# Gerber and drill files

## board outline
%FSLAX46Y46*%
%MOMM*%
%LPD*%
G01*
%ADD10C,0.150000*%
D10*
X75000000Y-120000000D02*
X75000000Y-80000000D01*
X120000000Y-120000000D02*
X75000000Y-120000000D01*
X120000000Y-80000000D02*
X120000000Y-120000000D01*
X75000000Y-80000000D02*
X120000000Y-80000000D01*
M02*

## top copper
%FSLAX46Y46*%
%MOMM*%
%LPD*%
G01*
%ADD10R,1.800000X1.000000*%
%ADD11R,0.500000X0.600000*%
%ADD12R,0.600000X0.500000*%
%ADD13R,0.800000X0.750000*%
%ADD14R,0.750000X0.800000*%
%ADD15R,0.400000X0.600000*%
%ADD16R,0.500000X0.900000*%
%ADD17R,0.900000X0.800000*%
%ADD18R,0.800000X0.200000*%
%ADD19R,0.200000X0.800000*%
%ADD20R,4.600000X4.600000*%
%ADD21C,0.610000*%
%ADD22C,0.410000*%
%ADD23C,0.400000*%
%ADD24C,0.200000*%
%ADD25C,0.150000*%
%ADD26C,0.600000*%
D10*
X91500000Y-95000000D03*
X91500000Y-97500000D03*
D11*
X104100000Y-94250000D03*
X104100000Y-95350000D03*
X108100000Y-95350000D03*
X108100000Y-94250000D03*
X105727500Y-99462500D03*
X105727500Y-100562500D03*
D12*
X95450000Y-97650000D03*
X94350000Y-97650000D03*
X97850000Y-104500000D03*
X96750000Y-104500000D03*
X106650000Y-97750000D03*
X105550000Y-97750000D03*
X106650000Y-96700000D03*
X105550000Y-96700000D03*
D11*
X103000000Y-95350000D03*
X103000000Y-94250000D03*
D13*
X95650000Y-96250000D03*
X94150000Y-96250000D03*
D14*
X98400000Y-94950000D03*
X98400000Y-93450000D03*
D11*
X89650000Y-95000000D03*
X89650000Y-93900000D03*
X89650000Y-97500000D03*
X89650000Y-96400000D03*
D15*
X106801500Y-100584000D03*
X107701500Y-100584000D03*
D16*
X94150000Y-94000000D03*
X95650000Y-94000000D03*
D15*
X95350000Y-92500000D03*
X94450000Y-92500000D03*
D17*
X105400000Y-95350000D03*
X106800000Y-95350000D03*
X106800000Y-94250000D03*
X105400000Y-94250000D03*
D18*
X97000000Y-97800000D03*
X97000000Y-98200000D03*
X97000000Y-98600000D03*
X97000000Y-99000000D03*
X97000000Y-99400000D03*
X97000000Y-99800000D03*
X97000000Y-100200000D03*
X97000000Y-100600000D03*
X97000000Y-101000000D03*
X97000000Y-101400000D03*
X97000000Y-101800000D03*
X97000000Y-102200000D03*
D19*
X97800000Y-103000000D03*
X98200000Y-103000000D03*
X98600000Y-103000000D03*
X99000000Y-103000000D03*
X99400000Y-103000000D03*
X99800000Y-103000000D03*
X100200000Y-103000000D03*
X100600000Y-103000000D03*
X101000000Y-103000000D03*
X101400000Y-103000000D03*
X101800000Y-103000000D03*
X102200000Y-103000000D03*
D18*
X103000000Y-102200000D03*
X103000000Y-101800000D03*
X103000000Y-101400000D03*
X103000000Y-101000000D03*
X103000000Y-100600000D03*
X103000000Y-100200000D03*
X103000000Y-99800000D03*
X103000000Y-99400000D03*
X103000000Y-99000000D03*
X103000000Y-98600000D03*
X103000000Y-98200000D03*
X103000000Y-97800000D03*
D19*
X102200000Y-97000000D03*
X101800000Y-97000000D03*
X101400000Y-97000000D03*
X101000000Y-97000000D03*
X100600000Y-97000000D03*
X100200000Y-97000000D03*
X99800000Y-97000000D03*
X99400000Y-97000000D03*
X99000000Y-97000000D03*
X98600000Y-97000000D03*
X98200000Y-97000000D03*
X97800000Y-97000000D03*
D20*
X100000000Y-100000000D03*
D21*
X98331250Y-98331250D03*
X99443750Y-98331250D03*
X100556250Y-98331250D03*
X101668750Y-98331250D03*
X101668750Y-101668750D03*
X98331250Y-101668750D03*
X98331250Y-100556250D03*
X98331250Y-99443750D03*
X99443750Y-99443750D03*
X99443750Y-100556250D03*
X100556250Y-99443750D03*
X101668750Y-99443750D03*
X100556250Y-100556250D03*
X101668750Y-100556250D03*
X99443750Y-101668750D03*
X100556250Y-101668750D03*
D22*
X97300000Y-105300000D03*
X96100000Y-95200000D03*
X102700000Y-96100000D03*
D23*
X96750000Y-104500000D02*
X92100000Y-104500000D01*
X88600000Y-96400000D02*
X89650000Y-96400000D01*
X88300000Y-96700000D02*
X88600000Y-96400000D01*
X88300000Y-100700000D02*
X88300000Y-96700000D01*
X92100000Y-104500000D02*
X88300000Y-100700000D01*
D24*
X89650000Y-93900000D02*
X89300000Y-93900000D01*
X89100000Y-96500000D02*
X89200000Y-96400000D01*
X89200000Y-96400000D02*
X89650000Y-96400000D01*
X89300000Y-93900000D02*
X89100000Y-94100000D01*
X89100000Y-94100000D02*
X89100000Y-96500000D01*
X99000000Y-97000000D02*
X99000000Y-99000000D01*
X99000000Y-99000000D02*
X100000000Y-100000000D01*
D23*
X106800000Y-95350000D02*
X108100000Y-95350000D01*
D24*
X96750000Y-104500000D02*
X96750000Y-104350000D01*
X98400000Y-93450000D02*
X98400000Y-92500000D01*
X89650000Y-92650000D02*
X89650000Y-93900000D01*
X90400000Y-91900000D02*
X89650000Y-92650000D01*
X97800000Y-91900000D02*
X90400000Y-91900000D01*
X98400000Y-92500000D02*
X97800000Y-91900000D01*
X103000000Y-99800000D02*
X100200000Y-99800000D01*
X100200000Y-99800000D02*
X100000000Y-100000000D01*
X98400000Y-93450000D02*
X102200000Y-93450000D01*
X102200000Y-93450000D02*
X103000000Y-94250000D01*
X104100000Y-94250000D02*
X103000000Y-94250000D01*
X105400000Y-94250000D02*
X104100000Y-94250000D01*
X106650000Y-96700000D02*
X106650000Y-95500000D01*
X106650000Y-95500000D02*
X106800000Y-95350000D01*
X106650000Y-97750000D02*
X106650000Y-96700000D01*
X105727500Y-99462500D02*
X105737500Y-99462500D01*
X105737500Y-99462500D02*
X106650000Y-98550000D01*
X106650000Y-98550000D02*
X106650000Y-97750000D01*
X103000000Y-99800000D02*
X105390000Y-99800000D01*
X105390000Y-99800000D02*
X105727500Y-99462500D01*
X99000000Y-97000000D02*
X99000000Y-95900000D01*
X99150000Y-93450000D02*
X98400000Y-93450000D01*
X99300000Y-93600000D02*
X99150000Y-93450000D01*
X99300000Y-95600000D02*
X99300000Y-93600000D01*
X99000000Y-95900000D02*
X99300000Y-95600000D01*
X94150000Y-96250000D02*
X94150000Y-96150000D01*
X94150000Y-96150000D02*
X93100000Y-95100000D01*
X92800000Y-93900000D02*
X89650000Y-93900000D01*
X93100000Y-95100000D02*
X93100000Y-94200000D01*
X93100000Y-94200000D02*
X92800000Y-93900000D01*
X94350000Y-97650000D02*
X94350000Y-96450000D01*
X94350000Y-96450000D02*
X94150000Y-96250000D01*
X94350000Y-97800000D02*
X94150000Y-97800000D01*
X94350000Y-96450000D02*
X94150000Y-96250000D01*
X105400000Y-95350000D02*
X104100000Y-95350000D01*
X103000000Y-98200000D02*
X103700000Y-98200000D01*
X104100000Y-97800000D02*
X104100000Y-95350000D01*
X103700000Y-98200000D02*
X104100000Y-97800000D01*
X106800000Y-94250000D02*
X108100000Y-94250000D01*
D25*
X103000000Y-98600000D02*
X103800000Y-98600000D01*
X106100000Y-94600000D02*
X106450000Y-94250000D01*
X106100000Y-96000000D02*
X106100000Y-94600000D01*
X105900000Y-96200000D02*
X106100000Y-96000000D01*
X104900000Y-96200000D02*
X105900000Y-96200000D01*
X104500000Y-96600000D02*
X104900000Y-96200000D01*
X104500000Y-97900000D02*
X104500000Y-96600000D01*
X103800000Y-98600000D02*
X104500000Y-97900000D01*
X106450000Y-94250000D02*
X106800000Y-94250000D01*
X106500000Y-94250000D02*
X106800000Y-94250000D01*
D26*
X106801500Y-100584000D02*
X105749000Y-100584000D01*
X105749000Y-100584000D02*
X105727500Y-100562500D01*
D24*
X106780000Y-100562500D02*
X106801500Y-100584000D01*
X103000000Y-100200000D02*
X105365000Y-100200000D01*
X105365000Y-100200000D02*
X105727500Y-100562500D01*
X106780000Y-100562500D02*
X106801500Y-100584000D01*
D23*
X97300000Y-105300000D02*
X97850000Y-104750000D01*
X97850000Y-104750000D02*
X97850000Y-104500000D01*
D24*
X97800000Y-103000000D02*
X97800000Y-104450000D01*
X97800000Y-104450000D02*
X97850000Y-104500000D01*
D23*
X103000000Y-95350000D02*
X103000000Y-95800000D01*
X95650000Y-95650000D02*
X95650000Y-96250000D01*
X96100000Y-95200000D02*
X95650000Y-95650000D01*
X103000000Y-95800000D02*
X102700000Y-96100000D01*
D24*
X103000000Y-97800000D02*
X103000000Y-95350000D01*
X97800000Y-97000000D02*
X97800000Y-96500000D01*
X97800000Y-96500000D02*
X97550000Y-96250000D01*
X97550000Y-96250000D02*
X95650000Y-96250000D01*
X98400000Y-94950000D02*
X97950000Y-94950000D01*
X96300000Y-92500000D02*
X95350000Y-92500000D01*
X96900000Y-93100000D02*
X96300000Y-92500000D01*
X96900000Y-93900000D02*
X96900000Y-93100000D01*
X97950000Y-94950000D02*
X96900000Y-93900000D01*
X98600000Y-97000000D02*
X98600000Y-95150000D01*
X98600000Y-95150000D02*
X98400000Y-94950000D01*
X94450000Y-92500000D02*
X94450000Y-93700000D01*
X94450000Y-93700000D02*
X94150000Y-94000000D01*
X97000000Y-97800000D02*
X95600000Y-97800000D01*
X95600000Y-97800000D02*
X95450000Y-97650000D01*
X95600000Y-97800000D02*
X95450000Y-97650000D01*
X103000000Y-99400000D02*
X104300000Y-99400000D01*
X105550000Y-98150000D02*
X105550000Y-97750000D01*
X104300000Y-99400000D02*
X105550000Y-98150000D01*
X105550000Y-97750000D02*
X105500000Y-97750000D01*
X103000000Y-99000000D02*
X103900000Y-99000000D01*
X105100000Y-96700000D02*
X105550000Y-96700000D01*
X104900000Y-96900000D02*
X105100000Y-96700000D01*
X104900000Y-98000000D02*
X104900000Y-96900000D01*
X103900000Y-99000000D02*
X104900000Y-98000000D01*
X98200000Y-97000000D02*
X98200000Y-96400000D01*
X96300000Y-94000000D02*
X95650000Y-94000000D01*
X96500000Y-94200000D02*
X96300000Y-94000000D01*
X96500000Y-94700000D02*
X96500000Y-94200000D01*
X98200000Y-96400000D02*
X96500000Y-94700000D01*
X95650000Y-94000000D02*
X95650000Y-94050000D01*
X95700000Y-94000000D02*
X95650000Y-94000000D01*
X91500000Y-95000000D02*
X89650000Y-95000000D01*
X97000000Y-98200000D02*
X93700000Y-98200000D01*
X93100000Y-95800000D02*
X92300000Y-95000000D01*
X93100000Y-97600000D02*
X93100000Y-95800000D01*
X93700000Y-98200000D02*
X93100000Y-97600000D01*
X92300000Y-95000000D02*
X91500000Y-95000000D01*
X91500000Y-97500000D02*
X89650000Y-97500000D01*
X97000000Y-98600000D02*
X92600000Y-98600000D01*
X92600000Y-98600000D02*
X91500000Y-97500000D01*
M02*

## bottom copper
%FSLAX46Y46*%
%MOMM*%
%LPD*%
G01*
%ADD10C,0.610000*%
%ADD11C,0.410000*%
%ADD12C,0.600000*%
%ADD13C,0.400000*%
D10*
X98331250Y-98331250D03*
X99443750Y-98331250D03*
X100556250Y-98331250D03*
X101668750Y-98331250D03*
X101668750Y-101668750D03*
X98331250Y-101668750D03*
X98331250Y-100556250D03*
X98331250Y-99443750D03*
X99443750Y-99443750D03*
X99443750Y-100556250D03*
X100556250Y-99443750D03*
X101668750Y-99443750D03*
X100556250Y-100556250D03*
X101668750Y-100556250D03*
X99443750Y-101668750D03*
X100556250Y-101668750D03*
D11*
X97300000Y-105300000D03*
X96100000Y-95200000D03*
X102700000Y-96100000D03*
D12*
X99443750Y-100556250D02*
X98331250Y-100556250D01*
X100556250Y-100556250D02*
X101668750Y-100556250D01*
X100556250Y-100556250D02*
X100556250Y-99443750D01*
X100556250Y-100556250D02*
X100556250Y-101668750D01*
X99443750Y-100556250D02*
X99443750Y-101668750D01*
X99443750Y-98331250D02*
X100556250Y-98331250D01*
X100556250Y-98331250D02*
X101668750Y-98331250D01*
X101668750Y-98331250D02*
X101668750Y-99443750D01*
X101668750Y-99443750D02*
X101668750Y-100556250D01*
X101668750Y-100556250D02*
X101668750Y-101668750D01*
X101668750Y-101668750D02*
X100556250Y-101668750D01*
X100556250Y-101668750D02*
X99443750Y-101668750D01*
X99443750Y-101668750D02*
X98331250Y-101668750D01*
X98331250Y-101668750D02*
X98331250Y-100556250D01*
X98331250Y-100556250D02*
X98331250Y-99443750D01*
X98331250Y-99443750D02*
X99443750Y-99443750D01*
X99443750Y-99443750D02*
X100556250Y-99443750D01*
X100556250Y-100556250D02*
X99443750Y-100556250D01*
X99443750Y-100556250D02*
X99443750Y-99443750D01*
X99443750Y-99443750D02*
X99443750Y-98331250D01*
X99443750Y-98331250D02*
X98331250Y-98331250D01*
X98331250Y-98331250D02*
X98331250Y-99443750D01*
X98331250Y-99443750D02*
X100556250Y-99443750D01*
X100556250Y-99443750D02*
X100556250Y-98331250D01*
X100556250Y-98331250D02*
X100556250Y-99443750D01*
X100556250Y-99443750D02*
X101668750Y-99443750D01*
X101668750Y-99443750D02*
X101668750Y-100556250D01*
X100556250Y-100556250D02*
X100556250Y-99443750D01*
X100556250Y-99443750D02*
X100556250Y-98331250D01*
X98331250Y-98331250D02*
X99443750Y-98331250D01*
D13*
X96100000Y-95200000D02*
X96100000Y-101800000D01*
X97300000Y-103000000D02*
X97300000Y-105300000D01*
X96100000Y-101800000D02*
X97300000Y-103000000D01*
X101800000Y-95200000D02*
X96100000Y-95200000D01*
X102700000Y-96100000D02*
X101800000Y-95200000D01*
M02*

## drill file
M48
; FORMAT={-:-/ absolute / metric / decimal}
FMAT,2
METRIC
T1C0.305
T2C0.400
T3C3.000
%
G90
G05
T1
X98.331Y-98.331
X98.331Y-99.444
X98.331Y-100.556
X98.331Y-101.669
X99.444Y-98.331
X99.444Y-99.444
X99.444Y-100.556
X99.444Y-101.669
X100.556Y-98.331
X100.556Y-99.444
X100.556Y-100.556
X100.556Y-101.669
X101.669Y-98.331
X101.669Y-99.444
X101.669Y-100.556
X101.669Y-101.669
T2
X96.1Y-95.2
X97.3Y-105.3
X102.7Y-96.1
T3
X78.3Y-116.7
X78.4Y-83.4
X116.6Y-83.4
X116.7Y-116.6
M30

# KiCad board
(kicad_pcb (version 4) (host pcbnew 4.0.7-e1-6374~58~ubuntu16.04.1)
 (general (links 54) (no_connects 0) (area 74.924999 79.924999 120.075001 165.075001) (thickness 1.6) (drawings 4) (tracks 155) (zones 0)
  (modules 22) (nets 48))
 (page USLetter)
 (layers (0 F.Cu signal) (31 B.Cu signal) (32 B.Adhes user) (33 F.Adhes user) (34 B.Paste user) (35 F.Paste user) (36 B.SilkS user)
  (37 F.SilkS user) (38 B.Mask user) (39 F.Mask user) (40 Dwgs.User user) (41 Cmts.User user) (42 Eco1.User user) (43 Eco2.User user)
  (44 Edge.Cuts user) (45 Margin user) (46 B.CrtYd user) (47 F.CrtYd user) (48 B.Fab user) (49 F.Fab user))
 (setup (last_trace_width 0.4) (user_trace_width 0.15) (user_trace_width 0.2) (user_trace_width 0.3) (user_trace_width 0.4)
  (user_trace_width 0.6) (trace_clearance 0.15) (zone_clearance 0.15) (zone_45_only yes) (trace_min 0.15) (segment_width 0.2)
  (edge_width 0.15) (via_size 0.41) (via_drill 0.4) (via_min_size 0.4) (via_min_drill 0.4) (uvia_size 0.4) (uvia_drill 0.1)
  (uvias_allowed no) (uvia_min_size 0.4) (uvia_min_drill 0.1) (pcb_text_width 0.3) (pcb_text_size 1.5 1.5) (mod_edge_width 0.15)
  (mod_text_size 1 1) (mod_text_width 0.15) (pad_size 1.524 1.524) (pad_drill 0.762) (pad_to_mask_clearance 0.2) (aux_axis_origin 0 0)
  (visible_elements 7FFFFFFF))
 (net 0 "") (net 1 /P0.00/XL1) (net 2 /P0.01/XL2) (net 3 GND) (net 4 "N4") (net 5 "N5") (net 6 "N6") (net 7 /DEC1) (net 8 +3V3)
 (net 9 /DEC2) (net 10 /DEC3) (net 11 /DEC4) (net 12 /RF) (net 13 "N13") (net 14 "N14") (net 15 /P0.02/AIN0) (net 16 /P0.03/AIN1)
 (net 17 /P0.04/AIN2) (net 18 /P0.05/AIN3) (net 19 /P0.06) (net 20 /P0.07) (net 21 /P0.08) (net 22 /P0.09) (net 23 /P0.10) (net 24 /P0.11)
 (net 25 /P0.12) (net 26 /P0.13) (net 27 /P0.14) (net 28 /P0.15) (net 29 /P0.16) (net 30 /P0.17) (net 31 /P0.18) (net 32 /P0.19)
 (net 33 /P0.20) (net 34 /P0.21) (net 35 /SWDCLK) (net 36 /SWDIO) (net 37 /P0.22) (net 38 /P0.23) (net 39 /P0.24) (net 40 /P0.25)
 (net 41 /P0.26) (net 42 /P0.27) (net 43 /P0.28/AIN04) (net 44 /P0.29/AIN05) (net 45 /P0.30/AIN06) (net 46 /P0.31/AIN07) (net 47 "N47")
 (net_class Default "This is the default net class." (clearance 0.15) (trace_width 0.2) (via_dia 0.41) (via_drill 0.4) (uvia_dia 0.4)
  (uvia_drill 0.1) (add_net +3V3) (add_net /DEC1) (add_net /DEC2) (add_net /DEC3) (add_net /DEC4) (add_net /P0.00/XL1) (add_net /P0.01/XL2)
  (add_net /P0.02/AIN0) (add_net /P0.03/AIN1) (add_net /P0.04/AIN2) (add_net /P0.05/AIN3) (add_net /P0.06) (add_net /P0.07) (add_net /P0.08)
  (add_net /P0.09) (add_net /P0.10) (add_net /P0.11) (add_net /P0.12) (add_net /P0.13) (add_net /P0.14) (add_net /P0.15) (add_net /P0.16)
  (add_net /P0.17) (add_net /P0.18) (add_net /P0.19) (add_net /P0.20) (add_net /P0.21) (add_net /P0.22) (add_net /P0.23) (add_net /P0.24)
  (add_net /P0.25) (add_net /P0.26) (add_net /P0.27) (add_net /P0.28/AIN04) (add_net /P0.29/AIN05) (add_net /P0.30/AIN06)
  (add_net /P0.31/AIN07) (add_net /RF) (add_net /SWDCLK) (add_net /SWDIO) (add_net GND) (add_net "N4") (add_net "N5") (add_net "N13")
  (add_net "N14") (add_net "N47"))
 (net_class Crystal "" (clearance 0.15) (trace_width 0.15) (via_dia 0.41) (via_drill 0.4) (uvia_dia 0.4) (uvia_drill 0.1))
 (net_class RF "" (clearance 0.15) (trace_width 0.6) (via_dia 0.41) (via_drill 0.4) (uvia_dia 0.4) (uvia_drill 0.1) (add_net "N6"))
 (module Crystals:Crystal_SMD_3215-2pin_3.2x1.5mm (layer F.Cu) (at 91.5 96.25 90)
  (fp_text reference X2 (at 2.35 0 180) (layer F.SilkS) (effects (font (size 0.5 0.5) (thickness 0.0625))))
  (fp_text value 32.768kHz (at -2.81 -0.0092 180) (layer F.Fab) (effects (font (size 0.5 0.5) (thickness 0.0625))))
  (pad 1 smd rect (at 1.25 0 90) (size 1 1.8) (layers F.Cu F.Paste F.Mask) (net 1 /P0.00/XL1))
  (pad 2 smd rect (at -1.25 0 90) (size 1 1.8) (layers F.Cu F.Paste F.Mask) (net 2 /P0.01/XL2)))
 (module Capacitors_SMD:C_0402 (layer F.Cu) (at 104.1 94.8 270)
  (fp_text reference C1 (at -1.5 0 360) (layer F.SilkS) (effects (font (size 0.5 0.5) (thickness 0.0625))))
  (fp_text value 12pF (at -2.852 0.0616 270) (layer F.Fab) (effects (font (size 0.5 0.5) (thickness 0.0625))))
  (pad 1 smd rect (at -0.55 0 270) (size 0.6 0.5) (layers F.Cu F.Paste F.Mask) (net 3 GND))
  (pad 2 smd rect (at 0.55 0 270) (size 0.6 0.5) (layers F.Cu F.Paste F.Mask) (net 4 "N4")))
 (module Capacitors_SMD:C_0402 (layer F.Cu) (at 108.1 94.8 90)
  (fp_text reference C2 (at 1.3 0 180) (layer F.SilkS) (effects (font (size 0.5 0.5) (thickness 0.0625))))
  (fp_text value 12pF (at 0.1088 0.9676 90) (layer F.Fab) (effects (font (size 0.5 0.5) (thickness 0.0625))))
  (pad 1 smd rect (at -0.55 0 90) (size 0.6 0.5) (layers F.Cu F.Paste F.Mask) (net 3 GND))
  (pad 2 smd rect (at 0.55 0 90) (size 0.6 0.5) (layers F.Cu F.Paste F.Mask) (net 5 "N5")))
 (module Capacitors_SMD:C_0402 (layer F.Cu) (at 105.7275 100.0125 270)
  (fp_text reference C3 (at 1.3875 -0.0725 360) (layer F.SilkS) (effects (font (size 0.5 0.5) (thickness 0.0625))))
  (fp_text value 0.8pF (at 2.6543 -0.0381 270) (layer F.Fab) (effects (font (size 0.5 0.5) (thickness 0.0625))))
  (pad 1 smd rect (at -0.55 0 270) (size 0.6 0.5) (layers F.Cu F.Paste F.Mask) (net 3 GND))
  (pad 2 smd rect (at 0.55 0 270) (size 0.6 0.5) (layers F.Cu F.Paste F.Mask) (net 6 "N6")))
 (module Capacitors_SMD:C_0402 (layer F.Cu) (at 94.9 97.65 180)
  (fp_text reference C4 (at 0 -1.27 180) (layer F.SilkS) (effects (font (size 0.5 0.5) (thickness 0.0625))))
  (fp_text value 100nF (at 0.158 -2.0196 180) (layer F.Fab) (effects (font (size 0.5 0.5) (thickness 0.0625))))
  (pad 1 smd rect (at -0.55 0 180) (size 0.6 0.5) (layers F.Cu F.Paste F.Mask) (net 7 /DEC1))
  (pad 2 smd rect (at 0.55 0 180) (size 0.6 0.5) (layers F.Cu F.Paste F.Mask) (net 3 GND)))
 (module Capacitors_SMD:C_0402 (layer F.Cu) (at 97.3 104.5 180)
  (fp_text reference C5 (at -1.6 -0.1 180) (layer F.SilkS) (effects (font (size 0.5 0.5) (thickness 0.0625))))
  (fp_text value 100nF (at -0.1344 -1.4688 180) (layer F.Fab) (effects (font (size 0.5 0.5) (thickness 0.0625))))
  (pad 1 smd rect (at -0.55 0 180) (size 0.6 0.5) (layers F.Cu F.Paste F.Mask) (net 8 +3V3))
  (pad 2 smd rect (at 0.55 0 180) (size 0.6 0.5) (layers F.Cu F.Paste F.Mask) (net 3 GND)))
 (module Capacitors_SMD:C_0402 (layer F.Cu) (at 106.1 97.75 180)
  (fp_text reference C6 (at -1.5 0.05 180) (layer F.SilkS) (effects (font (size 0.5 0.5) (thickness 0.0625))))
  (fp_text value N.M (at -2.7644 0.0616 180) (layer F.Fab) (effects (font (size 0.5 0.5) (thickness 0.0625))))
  (pad 1 smd rect (at -0.55 0 180) (size 0.6 0.5) (layers F.Cu F.Paste F.Mask) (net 3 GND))
  (pad 2 smd rect (at 0.55 0 180) (size 0.6 0.5) (layers F.Cu F.Paste F.Mask) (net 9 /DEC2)))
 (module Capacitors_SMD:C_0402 (layer F.Cu) (at 106.1 96.7 180)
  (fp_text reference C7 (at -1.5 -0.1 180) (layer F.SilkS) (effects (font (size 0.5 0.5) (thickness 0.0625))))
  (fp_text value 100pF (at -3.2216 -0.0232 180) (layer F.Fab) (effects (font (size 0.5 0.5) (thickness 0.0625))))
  (pad 1 smd rect (at -0.55 0 180) (size 0.6 0.5) (layers F.Cu F.Paste F.Mask) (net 3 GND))
  (pad 2 smd rect (at 0.55 0 180) (size 0.6 0.5) (layers F.Cu F.Paste F.Mask) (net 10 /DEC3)))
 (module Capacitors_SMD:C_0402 (layer F.Cu) (at 103 94.8 90)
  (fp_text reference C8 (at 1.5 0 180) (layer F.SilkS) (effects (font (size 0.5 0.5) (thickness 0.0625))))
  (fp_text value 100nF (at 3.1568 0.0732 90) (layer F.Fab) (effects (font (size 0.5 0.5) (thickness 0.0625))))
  (pad 1 smd rect (at -0.55 0 90) (size 0.6 0.5) (layers F.Cu F.Paste F.Mask) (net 8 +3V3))
  (pad 2 smd rect (at 0.55 0 90) (size 0.6 0.5) (layers F.Cu F.Paste F.Mask) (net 3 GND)))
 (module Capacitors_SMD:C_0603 (layer F.Cu) (at 94.9 96.25 180)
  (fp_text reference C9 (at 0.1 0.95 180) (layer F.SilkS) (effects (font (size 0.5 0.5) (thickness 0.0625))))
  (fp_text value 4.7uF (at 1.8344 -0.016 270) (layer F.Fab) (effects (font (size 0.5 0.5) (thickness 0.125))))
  (pad 1 smd rect (at -0.75 0 180) (size 0.8 0.75) (layers F.Cu F.Paste F.Mask) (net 8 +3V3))
  (pad 2 smd rect (at 0.75 0 180) (size 0.8 0.75) (layers F.Cu F.Paste F.Mask) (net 3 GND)))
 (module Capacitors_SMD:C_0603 (layer F.Cu) (at 98.4 94.2 90)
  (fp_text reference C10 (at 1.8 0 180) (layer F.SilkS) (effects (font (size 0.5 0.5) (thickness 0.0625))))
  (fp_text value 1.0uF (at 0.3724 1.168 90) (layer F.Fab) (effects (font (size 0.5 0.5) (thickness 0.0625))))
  (pad 1 smd rect (at -0.75 0 90) (size 0.8 0.75) (layers F.Cu F.Paste F.Mask) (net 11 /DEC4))
  (pad 2 smd rect (at 0.75 0 90) (size 0.8 0.75) (layers F.Cu F.Paste F.Mask) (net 3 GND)))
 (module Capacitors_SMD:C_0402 (layer F.Cu) (at 89.65 94.45 90)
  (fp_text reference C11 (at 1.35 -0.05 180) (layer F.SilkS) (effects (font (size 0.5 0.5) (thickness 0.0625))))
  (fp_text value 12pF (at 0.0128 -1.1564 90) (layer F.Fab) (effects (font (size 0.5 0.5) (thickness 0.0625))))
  (pad 1 smd rect (at -0.55 0 90) (size 0.6 0.5) (layers F.Cu F.Paste F.Mask) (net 1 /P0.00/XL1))
  (pad 2 smd rect (at 0.55 0 90) (size 0.6 0.5) (layers F.Cu F.Paste F.Mask) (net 3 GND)))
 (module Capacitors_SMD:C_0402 (layer F.Cu) (at 89.65 96.95 90)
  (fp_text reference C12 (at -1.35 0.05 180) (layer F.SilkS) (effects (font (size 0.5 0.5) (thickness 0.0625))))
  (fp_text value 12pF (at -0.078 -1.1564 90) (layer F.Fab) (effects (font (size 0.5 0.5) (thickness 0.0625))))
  (pad 1 smd rect (at -0.55 0 90) (size 0.6 0.5) (layers F.Cu F.Paste F.Mask) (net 2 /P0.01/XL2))
  (pad 2 smd rect (at 0.55 0 90) (size 0.6 0.5) (layers F.Cu F.Paste F.Mask) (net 3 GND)))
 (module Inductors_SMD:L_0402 (layer F.Cu) (at 107.2515 100.584)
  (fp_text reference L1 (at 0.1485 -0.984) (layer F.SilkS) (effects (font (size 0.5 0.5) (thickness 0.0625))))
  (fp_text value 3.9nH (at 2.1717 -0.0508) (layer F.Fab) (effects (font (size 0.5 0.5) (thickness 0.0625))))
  (pad 1 smd rect (at -0.45 0) (size 0.4 0.6) (layers F.Cu F.Paste F.Mask) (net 6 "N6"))
  (pad 2 smd rect (at 0.45 0) (size 0.4 0.6) (layers F.Cu F.Paste F.Mask) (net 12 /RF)))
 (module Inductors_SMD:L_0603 (layer F.Cu) (at 94.9 94)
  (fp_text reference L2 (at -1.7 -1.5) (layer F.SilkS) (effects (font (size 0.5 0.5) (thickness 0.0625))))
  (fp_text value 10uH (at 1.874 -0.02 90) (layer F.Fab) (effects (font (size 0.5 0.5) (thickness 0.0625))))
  (pad 1 smd rect (at -0.75 0) (size 0.5 0.9) (layers F.Cu F.Paste F.Mask) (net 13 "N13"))
  (pad 2 smd rect (at 0.75 0) (size 0.5 0.9) (layers F.Cu F.Paste F.Mask) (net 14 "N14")))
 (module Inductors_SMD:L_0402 (layer F.Cu) (at 94.9 92.5 180)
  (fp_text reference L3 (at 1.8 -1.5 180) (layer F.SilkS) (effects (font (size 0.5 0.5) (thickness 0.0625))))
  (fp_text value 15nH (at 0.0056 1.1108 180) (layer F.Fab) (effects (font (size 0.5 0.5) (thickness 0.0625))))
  (pad 1 smd rect (at -0.45 0 180) (size 0.4 0.6) (layers F.Cu F.Paste F.Mask) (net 11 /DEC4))
  (pad 2 smd rect (at 0.45 0 180) (size 0.4 0.6) (layers F.Cu F.Paste F.Mask) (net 13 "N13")))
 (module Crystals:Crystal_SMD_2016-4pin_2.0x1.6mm (layer F.Cu) (at 106.1 94.8)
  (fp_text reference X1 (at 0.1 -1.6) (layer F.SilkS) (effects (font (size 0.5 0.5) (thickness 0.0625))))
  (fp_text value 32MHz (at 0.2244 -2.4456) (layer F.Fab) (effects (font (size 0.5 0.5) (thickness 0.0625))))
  (pad 1 smd rect (at -0.7 0.55) (size 0.9 0.8) (layers F.Cu F.Paste F.Mask) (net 4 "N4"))
  (pad 2 smd rect (at 0.7 0.55) (size 0.9 0.8) (layers F.Cu F.Paste F.Mask) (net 3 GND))
  (pad 3 smd rect (at 0.7 -0.55) (size 0.9 0.8) (layers F.Cu F.Paste F.Mask) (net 5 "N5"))
  (pad 4 smd rect (at -0.7 -0.55) (size 0.9 0.8) (layers F.Cu F.Paste F.Mask) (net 3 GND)))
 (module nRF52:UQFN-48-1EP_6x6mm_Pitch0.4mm (layer F.Cu) (at 100 100)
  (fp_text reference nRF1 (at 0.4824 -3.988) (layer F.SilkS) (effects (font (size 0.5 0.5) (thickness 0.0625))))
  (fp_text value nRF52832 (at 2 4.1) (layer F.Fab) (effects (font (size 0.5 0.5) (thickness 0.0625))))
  (pad 1 smd rect (at -3 -2.2) (size 0.8 0.2) (layers F.Cu F.Paste F.Mask) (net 7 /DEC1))
  (pad 2 smd rect (at -3 -1.8) (size 0.8 0.2) (layers F.Cu F.Paste F.Mask) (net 1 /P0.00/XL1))
  (pad 3 smd rect (at -3 -1.4) (size 0.8 0.2) (layers F.Cu F.Paste F.Mask) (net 2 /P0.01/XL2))
  (pad 4 smd rect (at -3 -1) (size 0.8 0.2) (layers F.Cu F.Paste F.Mask) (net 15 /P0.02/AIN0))
  (pad 5 smd rect (at -3 -0.6) (size 0.8 0.2) (layers F.Cu F.Paste F.Mask) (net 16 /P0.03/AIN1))
  (pad 6 smd rect (at -3 -0.2) (size 0.8 0.2) (layers F.Cu F.Paste F.Mask) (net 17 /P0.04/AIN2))
  (pad 7 smd rect (at -3 0.2) (size 0.8 0.2) (layers F.Cu F.Paste F.Mask) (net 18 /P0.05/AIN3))
  (pad 8 smd rect (at -3 0.6) (size 0.8 0.2) (layers F.Cu F.Paste F.Mask) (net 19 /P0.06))
  (pad 9 smd rect (at -3 1) (size 0.8 0.2) (layers F.Cu F.Paste F.Mask) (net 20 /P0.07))
  (pad 10 smd rect (at -3 1.4) (size 0.8 0.2) (layers F.Cu F.Paste F.Mask) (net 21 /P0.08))
  (pad 11 smd rect (at -3 1.8) (size 0.8 0.2) (layers F.Cu F.Paste F.Mask) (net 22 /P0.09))
  (pad 12 smd rect (at -3 2.2) (size 0.8 0.2) (layers F.Cu F.Paste F.Mask) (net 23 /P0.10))
  (pad 13 smd rect (at -2.2 3 90) (size 0.8 0.2) (layers F.Cu F.Paste F.Mask) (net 8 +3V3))
  (pad 14 smd rect (at -1.8 3 90) (size 0.8 0.2) (layers F.Cu F.Paste F.Mask) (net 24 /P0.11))
  (pad 15 smd rect (at -1.4 3 90) (size 0.8 0.2) (layers F.Cu F.Paste F.Mask) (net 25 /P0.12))
  (pad 16 smd rect (at -1 3 90) (size 0.8 0.2) (layers F.Cu F.Paste F.Mask) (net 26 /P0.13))
  (pad 17 smd rect (at -0.6 3 90) (size 0.8 0.2) (layers F.Cu F.Paste F.Mask) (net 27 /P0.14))
  (pad 18 smd rect (at -0.2 3 90) (size 0.8 0.2) (layers F.Cu F.Paste F.Mask) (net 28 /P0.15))
  (pad 19 smd rect (at 0.2 3 90) (size 0.8 0.2) (layers F.Cu F.Paste F.Mask) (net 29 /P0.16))
  (pad 20 smd rect (at 0.6 3 90) (size 0.8 0.2) (layers F.Cu F.Paste F.Mask) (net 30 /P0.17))
  (pad 21 smd rect (at 1 3 90) (size 0.8 0.2) (layers F.Cu F.Paste F.Mask) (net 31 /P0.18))
  (pad 22 smd rect (at 1.4 3 90) (size 0.8 0.2) (layers F.Cu F.Paste F.Mask) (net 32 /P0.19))
  (pad 23 smd rect (at 1.8 3 90) (size 0.8 0.2) (layers F.Cu F.Paste F.Mask) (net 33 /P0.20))
  (pad 24 smd rect (at 2.2 3 90) (size 0.8 0.2) (layers F.Cu F.Paste F.Mask) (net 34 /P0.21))
  (pad 25 smd rect (at 3 2.2) (size 0.8 0.2) (layers F.Cu F.Paste F.Mask) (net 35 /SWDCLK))
  (pad 26 smd rect (at 3 1.8) (size 0.8 0.2) (layers F.Cu F.Paste F.Mask) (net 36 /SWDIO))
  (pad 27 smd rect (at 3 1.4) (size 0.8 0.2) (layers F.Cu F.Paste F.Mask) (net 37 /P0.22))
  (pad 28 smd rect (at 3 1) (size 0.8 0.2) (layers F.Cu F.Paste F.Mask) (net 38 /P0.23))
  (pad 29 smd rect (at 3 0.6) (size 0.8 0.2) (layers F.Cu F.Paste F.Mask) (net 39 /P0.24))
  (pad 30 smd rect (at 3 0.2) (size 0.8 0.2) (layers F.Cu F.Paste F.Mask) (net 6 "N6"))
  (pad 31 smd rect (at 3 -0.2) (size 0.8 0.2) (layers F.Cu F.Paste F.Mask) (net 3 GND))
  (pad 32 smd rect (at 3 -0.6) (size 0.8 0.2) (layers F.Cu F.Paste F.Mask) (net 9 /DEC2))
  (pad 33 smd rect (at 3 -1) (size 0.8 0.2) (layers F.Cu F.Paste F.Mask) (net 10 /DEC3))
  (pad 34 smd rect (at 3 -1.4) (size 0.8 0.2) (layers F.Cu F.Paste F.Mask) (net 5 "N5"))
  (pad 35 smd rect (at 3 -1.8) (size 0.8 0.2) (layers F.Cu F.Paste F.Mask) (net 4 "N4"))
  (pad 36 smd rect (at 3 -2.2) (size 0.8 0.2) (layers F.Cu F.Paste F.Mask) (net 8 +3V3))
  (pad 37 smd rect (at 2.2 -3 90) (size 0.8 0.2) (layers F.Cu F.Paste F.Mask) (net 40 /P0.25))
  (pad 38 smd rect (at 1.8 -3 90) (size 0.8 0.2) (layers F.Cu F.Paste F.Mask) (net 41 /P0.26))
  (pad 39 smd rect (at 1.4 -3 90) (size 0.8 0.2) (layers F.Cu F.Paste F.Mask) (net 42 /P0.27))
  (pad 40 smd rect (at 1 -3 90) (size 0.8 0.2) (layers F.Cu F.Paste F.Mask) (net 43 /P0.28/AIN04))
  (pad 41 smd rect (at 0.6 -3 90) (size 0.8 0.2) (layers F.Cu F.Paste F.Mask) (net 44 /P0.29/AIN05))
  (pad 42 smd rect (at 0.2 -3 90) (size 0.8 0.2) (layers F.Cu F.Paste F.Mask) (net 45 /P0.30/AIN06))
  (pad 43 smd rect (at -0.2 -3 90) (size 0.8 0.2) (layers F.Cu F.Paste F.Mask) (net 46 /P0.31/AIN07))
  (pad 44 smd rect (at -0.6 -3 90) (size 0.8 0.2) (layers F.Cu F.Paste F.Mask) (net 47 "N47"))
  (pad 45 smd rect (at -1 -3 90) (size 0.8 0.2) (layers F.Cu F.Paste F.Mask) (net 3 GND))
  (pad 46 smd rect (at -1.4 -3 90) (size 0.8 0.2) (layers F.Cu F.Paste F.Mask) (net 11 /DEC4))
  (pad 47 smd rect (at -1.8 -3 90) (size 0.8 0.2) (layers F.Cu F.Paste F.Mask) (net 14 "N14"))
  (pad 48 smd rect (at -2.2 -3 90) (size 0.8 0.2) (layers F.Cu F.Paste F.Mask) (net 8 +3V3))
  (pad 49 smd rect (at 0 0) (size 4.6 4.6) (layers F.Cu F.Paste F.Mask) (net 3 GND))
  (pad 49 thru_hole circle (at -1.66875 -1.66875) (size 0.61 0.61) (drill 0.305) (layers *.Cu B.Mask) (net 3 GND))
  (pad 49 thru_hole circle (at -0.55625 -1.66875) (size 0.61 0.61) (drill 0.305) (layers *.Cu B.Mask) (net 3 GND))
  (pad 49 thru_hole circle (at 0.55625 -1.66875) (size 0.61 0.61) (drill 0.305) (layers *.Cu B.Mask) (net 3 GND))
  (pad 49 thru_hole circle (at 1.66875 -1.66875) (size 0.61 0.61) (drill 0.305) (layers *.Cu B.Mask) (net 3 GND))
  (pad 49 thru_hole circle (at 1.66875 1.66875) (size 0.61 0.61) (drill 0.305) (layers *.Cu B.Mask) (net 3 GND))
  (pad 49 thru_hole circle (at -1.66875 1.66875) (size 0.61 0.61) (drill 0.305) (layers *.Cu B.Mask) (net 3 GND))
  (pad 49 thru_hole circle (at -1.66875 0.55625) (size 0.61 0.61) (drill 0.305) (layers *.Cu B.Mask) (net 3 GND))
  (pad 49 thru_hole circle (at -1.66875 -0.55625) (size 0.61 0.61) (drill 0.305) (layers *.Cu B.Mask) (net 3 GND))
  (pad 49 thru_hole circle (at -0.55625 -0.55625) (size 0.61 0.61) (drill 0.305) (layers *.Cu B.Mask) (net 3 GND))
  (pad 49 thru_hole circle (at -0.55625 0.55625) (size 0.61 0.61) (drill 0.305) (layers *.Cu B.Mask) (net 3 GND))
  (pad 49 thru_hole circle (at 0.55625 -0.55625) (size 0.61 0.61) (drill 0.305) (layers *.Cu B.Mask) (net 3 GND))
  (pad 49 thru_hole circle (at 1.66875 -0.55625) (size 0.61 0.61) (drill 0.305) (layers *.Cu B.Mask) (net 3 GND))
  (pad 49 thru_hole circle (at 0.55625 0.55625) (size 0.61 0.61) (drill 0.305) (layers *.Cu B.Mask) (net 3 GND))
  (pad 49 thru_hole circle (at 1.66875 0.55625) (size 0.61 0.61) (drill 0.305) (layers *.Cu B.Mask) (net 3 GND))
  (pad 49 thru_hole circle (at -0.55625 1.66875) (size 0.61 0.61) (drill 0.305) (layers *.Cu B.Mask) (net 3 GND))
  (pad 49 thru_hole circle (at 0.55625 1.66875) (size 0.61 0.61) (drill 0.305) (layers *.Cu B.Mask) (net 3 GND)))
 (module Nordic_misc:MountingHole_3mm (layer F.Cu) (at 78.3 116.7)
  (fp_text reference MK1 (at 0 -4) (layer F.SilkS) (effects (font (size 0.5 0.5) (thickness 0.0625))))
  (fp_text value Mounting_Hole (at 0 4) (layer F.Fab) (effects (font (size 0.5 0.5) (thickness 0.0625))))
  (pad 1 np_thru_hole circle (at 0 0) (size 3 3) (drill 3) (layers *.Cu *.Mask)))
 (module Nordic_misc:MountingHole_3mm (layer F.Cu) (at 116.7 116.6)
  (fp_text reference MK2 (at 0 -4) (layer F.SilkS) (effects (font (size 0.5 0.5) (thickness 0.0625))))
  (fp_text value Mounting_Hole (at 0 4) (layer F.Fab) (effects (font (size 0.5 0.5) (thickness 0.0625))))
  (pad 1 np_thru_hole circle (at 0 0) (size 3 3) (drill 3) (layers *.Cu *.Mask)))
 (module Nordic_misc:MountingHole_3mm (layer F.Cu) (at 116.6 83.4)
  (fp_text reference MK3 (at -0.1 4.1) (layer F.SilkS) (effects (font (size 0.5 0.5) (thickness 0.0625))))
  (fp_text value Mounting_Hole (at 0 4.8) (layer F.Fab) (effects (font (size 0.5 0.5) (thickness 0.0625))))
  (pad 1 np_thru_hole circle (at 0 0) (size 3 3) (drill 3) (layers *.Cu *.Mask)))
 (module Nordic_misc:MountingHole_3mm (layer F.Cu) (at 78.4 83.4)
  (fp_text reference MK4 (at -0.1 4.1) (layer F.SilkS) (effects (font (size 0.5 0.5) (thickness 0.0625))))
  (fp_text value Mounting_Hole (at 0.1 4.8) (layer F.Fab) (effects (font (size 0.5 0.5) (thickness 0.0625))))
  (pad 1 np_thru_hole circle (at 0 0) (size 3 3) (drill 3) (layers *.Cu *.Mask)))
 (gr_line (start 75 120) (end 75 80) (angle 90) (layer Edge.Cuts) (width 0.15))
 (gr_line (start 120 120) (end 75 120) (angle 90) (layer Edge.Cuts) (width 0.15))
 (gr_line (start 120 80) (end 120 120) (angle 90) (layer Edge.Cuts) (width 0.15))
 (gr_line (start 75 80) (end 120 80) (angle 90) (layer Edge.Cuts) (width 0.15))
 (segment (start 96.75 104.5) (end 92.1 104.5) (width 0.4) (layer F.Cu) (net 3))
 (segment (start 88.6 96.4) (end 89.65 96.4) (width 0.4) (layer F.Cu) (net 3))
 (segment (start 88.3 96.7) (end 88.6 96.4) (width 0.4) (layer F.Cu) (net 3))
 (segment (start 88.3 100.7) (end 88.3 96.7) (width 0.4) (layer F.Cu) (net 3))
 (segment (start 92.1 104.5) (end 88.3 100.7) (width 0.4) (layer F.Cu) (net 3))
 (segment (start 89.65 93.9) (end 89.3 93.9) (width 0.2) (layer F.Cu) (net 3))
 (segment (start 89.1 96.5) (end 89.2 96.4) (width 0.2) (layer F.Cu) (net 3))
 (segment (start 89.2 96.4) (end 89.65 96.4) (width 0.2) (layer F.Cu) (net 3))
 (segment (start 89.3 93.9) (end 89.1 94.1) (width 0.2) (layer F.Cu) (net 3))
 (segment (start 89.1 94.1) (end 89.1 96.5) (width 0.2) (layer F.Cu) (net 3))
 (segment (start 99 97) (end 99 99) (width 0.2) (layer F.Cu) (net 3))
 (segment (start 99 99) (end 100 100) (width 0.2) (layer F.Cu) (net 3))
 (segment (start 106.8 95.35) (end 108.1 95.35) (width 0.4) (layer F.Cu) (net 3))
 (segment (start 96.75 104.5) (end 96.75 104.35) (width 0.2) (layer F.Cu) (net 3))
 (segment (start 98.4 93.45) (end 98.4 92.5) (width 0.2) (layer F.Cu) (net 3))
 (segment (start 89.65 92.65) (end 89.65 93.9) (width 0.2) (layer F.Cu) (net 3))
 (segment (start 90.4 91.9) (end 89.65 92.65) (width 0.2) (layer F.Cu) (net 3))
 (segment (start 97.8 91.9) (end 90.4 91.9) (width 0.2) (layer F.Cu) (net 3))
 (segment (start 98.4 92.5) (end 97.8 91.9) (width 0.2) (layer F.Cu) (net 3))
 (segment (start 99.44375 100.55625) (end 98.33125 100.55625) (width 0.6) (layer B.Cu) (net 3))
 (segment (start 100.55625 100.55625) (end 101.66875 100.55625) (width 0.6) (layer B.Cu) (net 3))
 (segment (start 100.55625 100.55625) (end 100.55625 99.44375) (width 0.6) (layer B.Cu) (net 3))
 (segment (start 100.55625 100.55625) (end 100.55625 101.66875) (width 0.6) (layer B.Cu) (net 3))
 (segment (start 99.44375 100.55625) (end 99.44375 101.66875) (width 0.6) (layer B.Cu) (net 3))
 (segment (start 99.44375 98.33125) (end 100.55625 98.33125) (width 0.6) (layer B.Cu) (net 3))
 (segment (start 100.55625 98.33125) (end 101.66875 98.33125) (width 0.6) (layer B.Cu) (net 3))
 (segment (start 101.66875 98.33125) (end 101.66875 99.44375) (width 0.6) (layer B.Cu) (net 3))
 (segment (start 101.66875 99.44375) (end 101.66875 100.55625) (width 0.6) (layer B.Cu) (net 3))
 (segment (start 101.66875 100.55625) (end 101.66875 101.66875) (width 0.6) (layer B.Cu) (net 3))
 (segment (start 101.66875 101.66875) (end 100.55625 101.66875) (width 0.6) (layer B.Cu) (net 3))
 (segment (start 100.55625 101.66875) (end 99.44375 101.66875) (width 0.6) (layer B.Cu) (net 3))
 (segment (start 99.44375 101.66875) (end 98.33125 101.66875) (width 0.6) (layer B.Cu) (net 3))
 (segment (start 98.33125 101.66875) (end 98.33125 100.55625) (width 0.6) (layer B.Cu) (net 3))
 (segment (start 98.33125 100.55625) (end 98.33125 99.44375) (width 0.6) (layer B.Cu) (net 3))
 (segment (start 98.33125 99.44375) (end 99.44375 99.44375) (width 0.6) (layer B.Cu) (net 3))
 (segment (start 99.44375 99.44375) (end 100.55625 99.44375) (width 0.6) (layer B.Cu) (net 3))
 (segment (start 100.55625 100.55625) (end 99.44375 100.55625) (width 0.6) (layer B.Cu) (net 3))
 (segment (start 99.44375 100.55625) (end 99.44375 99.44375) (width 0.6) (layer B.Cu) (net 3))
 (segment (start 99.44375 99.44375) (end 99.44375 98.33125) (width 0.6) (layer B.Cu) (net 3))
 (segment (start 99.44375 98.33125) (end 98.33125 98.33125) (width 0.6) (layer B.Cu) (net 3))
 (segment (start 98.33125 98.33125) (end 98.33125 99.44375) (width 0.6) (layer B.Cu) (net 3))
 (segment (start 98.33125 99.44375) (end 100.55625 99.44375) (width 0.6) (layer B.Cu) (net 3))
 (segment (start 100.55625 99.44375) (end 100.55625 98.33125) (width 0.6) (layer B.Cu) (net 3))
 (segment (start 100.55625 98.33125) (end 100.55625 99.44375) (width 0.6) (layer B.Cu) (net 3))
 (segment (start 100.55625 99.44375) (end 101.66875 99.44375) (width 0.6) (layer B.Cu) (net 3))
 (segment (start 101.66875 99.44375) (end 101.66875 100.55625) (width 0.6) (layer B.Cu) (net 3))
 (segment (start 100.55625 100.55625) (end 100.55625 99.44375) (width 0.6) (layer B.Cu) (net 3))
 (segment (start 100.55625 99.44375) (end 100.55625 98.33125) (width 0.6) (layer B.Cu) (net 3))
 (segment (start 98.33125 98.33125) (end 99.44375 98.33125) (width 0.6) (layer B.Cu) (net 3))
 (segment (start 103 99.8) (end 100.2 99.8) (width 0.2) (layer F.Cu) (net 3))
 (segment (start 100.2 99.8) (end 100 100) (width 0.2) (layer F.Cu) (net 3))
 (segment (start 98.4 93.45) (end 102.2 93.45) (width 0.2) (layer F.Cu) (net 3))
 (segment (start 102.2 93.45) (end 103 94.25) (width 0.2) (layer F.Cu) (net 3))
 (segment (start 104.1 94.25) (end 103 94.25) (width 0.2) (layer F.Cu) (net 3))
 (segment (start 105.4 94.25) (end 104.1 94.25) (width 0.2) (layer F.Cu) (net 3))
 (segment (start 106.65 96.7) (end 106.65 95.5) (width 0.2) (layer F.Cu) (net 3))
 (segment (start 106.65 95.5) (end 106.8 95.35) (width 0.2) (layer F.Cu) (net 3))
 (segment (start 106.65 97.75) (end 106.65 96.7) (width 0.2) (layer F.Cu) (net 3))
 (segment (start 105.7275 99.4625) (end 105.7375 99.4625) (width 0.2) (layer F.Cu) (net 3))
 (segment (start 105.7375 99.4625) (end 106.65 98.55) (width 0.2) (layer F.Cu) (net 3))
 (segment (start 106.65 98.55) (end 106.65 97.75) (width 0.2) (layer F.Cu) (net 3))
 (segment (start 103 99.8) (end 105.39 99.8) (width 0.2) (layer F.Cu) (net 3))
 (segment (start 105.39 99.8) (end 105.7275 99.4625) (width 0.2) (layer F.Cu) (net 3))
 (segment (start 99 97) (end 99 95.9) (width 0.2) (layer F.Cu) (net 3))
 (segment (start 99.15 93.45) (end 98.4 93.45) (width 0.2) (layer F.Cu) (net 3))
 (segment (start 99.3 93.6) (end 99.15 93.45) (width 0.2) (layer F.Cu) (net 3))
 (segment (start 99.3 95.6) (end 99.3 93.6) (width 0.2) (layer F.Cu) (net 3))
 (segment (start 99 95.9) (end 99.3 95.6) (width 0.2) (layer F.Cu) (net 3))
 (segment (start 94.15 96.25) (end 94.15 96.15) (width 0.2) (layer F.Cu) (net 3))
 (segment (start 94.15 96.15) (end 93.1 95.1) (width 0.2) (layer F.Cu) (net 3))
 (segment (start 92.8 93.9) (end 89.65 93.9) (width 0.2) (layer F.Cu) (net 3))
 (segment (start 93.1 95.1) (end 93.1 94.2) (width 0.2) (layer F.Cu) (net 3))
 (segment (start 93.1 94.2) (end 92.8 93.9) (width 0.2) (layer F.Cu) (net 3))
 (segment (start 94.35 97.65) (end 94.35 96.45) (width 0.2) (layer F.Cu) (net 3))
 (segment (start 94.35 96.45) (end 94.15 96.25) (width 0.2) (layer F.Cu) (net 3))
 (segment (start 94.35 97.8) (end 94.15 97.8) (width 0.2) (layer F.Cu) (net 3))
 (segment (start 94.35 96.45) (end 94.15 96.25) (width 0.2) (layer F.Cu) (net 3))
 (segment (start 105.4 95.35) (end 104.1 95.35) (width 0.2) (layer F.Cu) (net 4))
 (segment (start 103 98.2) (end 103.7 98.2) (width 0.2) (layer F.Cu) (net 4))
 (segment (start 104.1 97.8) (end 104.1 95.35) (width 0.2) (layer F.Cu) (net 4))
 (segment (start 103.7 98.2) (end 104.1 97.8) (width 0.2) (layer F.Cu) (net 4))
 (segment (start 106.8 94.25) (end 108.1 94.25) (width 0.2) (layer F.Cu) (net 5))
 (segment (start 103 98.6) (end 103.8 98.6) (width 0.15) (layer F.Cu) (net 5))
 (segment (start 106.1 94.6) (end 106.45 94.25) (width 0.15) (layer F.Cu) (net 5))
 (segment (start 106.1 96) (end 106.1 94.6) (width 0.15) (layer F.Cu) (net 5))
 (segment (start 105.9 96.2) (end 106.1 96) (width 0.15) (layer F.Cu) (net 5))
 (segment (start 104.9 96.2) (end 105.9 96.2) (width 0.15) (layer F.Cu) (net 5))
 (segment (start 104.5 96.6) (end 104.9 96.2) (width 0.15) (layer F.Cu) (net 5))
 (segment (start 104.5 97.9) (end 104.5 96.6) (width 0.15) (layer F.Cu) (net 5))
 (segment (start 103.8 98.6) (end 104.5 97.9) (width 0.15) (layer F.Cu) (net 5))
 (segment (start 106.45 94.25) (end 106.8 94.25) (width 0.15) (layer F.Cu) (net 5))
 (segment (start 106.5 94.25) (end 106.8 94.25) (width 0.15) (layer F.Cu) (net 5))
 (segment (start 106.8015 100.584) (end 105.749 100.584) (width 0.6) (layer F.Cu) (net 6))
 (segment (start 105.749 100.584) (end 105.7275 100.5625) (width 0.6) (layer F.Cu) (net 6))
 (segment (start 106.78 100.5625) (end 106.8015 100.584) (width 0.2) (layer F.Cu) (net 6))
 (segment (start 103 100.2) (end 105.365 100.2) (width 0.2) (layer F.Cu) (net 6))
 (segment (start 105.365 100.2) (end 105.7275 100.5625) (width 0.2) (layer F.Cu) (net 6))
 (segment (start 106.78 100.5625) (end 106.8015 100.584) (width 0.2) (layer F.Cu) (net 6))
 (segment (start 96.1 95.2) (end 96.1 101.8) (width 0.4) (layer B.Cu) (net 8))
 (segment (start 97.3 105.3) (end 97.85 104.75) (width 0.4) (layer F.Cu) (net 8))
 (via (at 97.3 105.3) (size 0.41) (drill 0.4) (layers F.Cu B.Cu) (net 8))
 (segment (start 97.3 103) (end 97.3 105.3) (width 0.4) (layer B.Cu) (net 8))
 (segment (start 96.1 101.8) (end 97.3 103) (width 0.4) (layer B.Cu) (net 8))
 (segment (start 97.85 104.75) (end 97.85 104.5) (width 0.4) (layer F.Cu) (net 8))
 (segment (start 97.8 103) (end 97.8 104.45) (width 0.2) (layer F.Cu) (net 8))
 (segment (start 97.8 104.45) (end 97.85 104.5) (width 0.2) (layer F.Cu) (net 8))
 (segment (start 103 95.35) (end 103 95.8) (width 0.4) (layer F.Cu) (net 8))
 (segment (start 95.65 95.65) (end 95.65 96.25) (width 0.4) (layer F.Cu) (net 8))
 (segment (start 96.1 95.2) (end 95.65 95.65) (width 0.4) (layer F.Cu) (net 8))
 (via (at 96.1 95.2) (size 0.41) (drill 0.4) (layers F.Cu B.Cu) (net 8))
 (segment (start 101.8 95.2) (end 96.1 95.2) (width 0.4) (layer B.Cu) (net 8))
 (segment (start 102.7 96.1) (end 101.8 95.2) (width 0.4) (layer B.Cu) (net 8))
 (via (at 102.7 96.1) (size 0.41) (drill 0.4) (layers F.Cu B.Cu) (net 8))
 (segment (start 103 95.8) (end 102.7 96.1) (width 0.4) (layer F.Cu) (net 8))
 (segment (start 103 97.8) (end 103 95.35) (width 0.2) (layer F.Cu) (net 8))
 (segment (start 97.8 97) (end 97.8 96.5) (width 0.2) (layer F.Cu) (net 8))
 (segment (start 97.8 96.5) (end 97.55 96.25) (width 0.2) (layer F.Cu) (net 8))
 (segment (start 97.55 96.25) (end 95.65 96.25) (width 0.2) (layer F.Cu) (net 8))
 (segment (start 98.4 94.95) (end 97.95 94.95) (width 0.2) (layer F.Cu) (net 11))
 (segment (start 96.3 92.5) (end 95.35 92.5) (width 0.2) (layer F.Cu) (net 11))
 (segment (start 96.9 93.1) (end 96.3 92.5) (width 0.2) (layer F.Cu) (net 11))
 (segment (start 96.9 93.9) (end 96.9 93.1) (width 0.2) (layer F.Cu) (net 11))
 (segment (start 97.95 94.95) (end 96.9 93.9) (width 0.2) (layer F.Cu) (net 11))
 (segment (start 98.6 97) (end 98.6 95.15) (width 0.2) (layer F.Cu) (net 11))
 (segment (start 98.6 95.15) (end 98.4 94.95) (width 0.2) (layer F.Cu) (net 11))
 (segment (start 94.45 92.5) (end 94.45 93.7) (width 0.2) (layer F.Cu) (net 13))
 (segment (start 94.45 93.7) (end 94.15 94) (width 0.2) (layer F.Cu) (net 13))
 (segment (start 97 97.8) (end 95.6 97.8) (width 0.2) (layer F.Cu) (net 7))
 (segment (start 95.6 97.8) (end 95.45 97.65) (width 0.2) (layer F.Cu) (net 7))
 (segment (start 95.6 97.8) (end 95.45 97.65) (width 0.2) (layer F.Cu) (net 7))
 (segment (start 103 99.4) (end 104.3 99.4) (width 0.2) (layer F.Cu) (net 9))
 (segment (start 105.55 98.15) (end 105.55 97.75) (width 0.2) (layer F.Cu) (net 9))
 (segment (start 104.3 99.4) (end 105.55 98.15) (width 0.2) (layer F.Cu) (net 9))
 (segment (start 105.55 97.75) (end 105.5 97.75) (width 0.2) (layer F.Cu) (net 9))
 (segment (start 103 99) (end 103.9 99) (width 0.2) (layer F.Cu) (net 10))
 (segment (start 105.1 96.7) (end 105.55 96.7) (width 0.2) (layer F.Cu) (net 10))
 (segment (start 104.9 96.9) (end 105.1 96.7) (width 0.2) (layer F.Cu) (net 10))
 (segment (start 104.9 98) (end 104.9 96.9) (width 0.2) (layer F.Cu) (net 10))
 (segment (start 103.9 99) (end 104.9 98) (width 0.2) (layer F.Cu) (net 10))
 (segment (start 98.2 97) (end 98.2 96.4) (width 0.2) (layer F.Cu) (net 14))
 (segment (start 96.3 94) (end 95.65 94) (width 0.2) (layer F.Cu) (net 14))
 (segment (start 96.5 94.2) (end 96.3 94) (width 0.2) (layer F.Cu) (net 14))
 (segment (start 96.5 94.7) (end 96.5 94.2) (width 0.2) (layer F.Cu) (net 14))
 (segment (start 98.2 96.4) (end 96.5 94.7) (width 0.2) (layer F.Cu) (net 14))
 (segment (start 95.65 94) (end 95.65 94.05) (width 0.2) (layer F.Cu) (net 14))
 (segment (start 95.7 94) (end 95.65 94) (width 0.2) (layer F.Cu) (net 14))
 (segment (start 91.5 95) (end 89.65 95) (width 0.2) (layer F.Cu) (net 1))
 (segment (start 97 98.2) (end 93.7 98.2) (width 0.2) (layer F.Cu) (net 1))
 (segment (start 93.1 95.8) (end 92.3 95) (width 0.2) (layer F.Cu) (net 1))
 (segment (start 93.1 97.6) (end 93.1 95.8) (width 0.2) (layer F.Cu) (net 1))
 (segment (start 93.7 98.2) (end 93.1 97.6) (width 0.2) (layer F.Cu) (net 1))
 (segment (start 92.3 95) (end 91.5 95) (width 0.2) (layer F.Cu) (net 1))
 (segment (start 91.5 97.5) (end 89.65 97.5) (width 0.2) (layer F.Cu) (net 2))
 (segment (start 97 98.6) (end 92.6 98.6) (width 0.2) (layer F.Cu) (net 2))
 (segment (start 92.6 98.6) (end 91.5 97.5) (width 0.2) (layer F.Cu) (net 2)))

